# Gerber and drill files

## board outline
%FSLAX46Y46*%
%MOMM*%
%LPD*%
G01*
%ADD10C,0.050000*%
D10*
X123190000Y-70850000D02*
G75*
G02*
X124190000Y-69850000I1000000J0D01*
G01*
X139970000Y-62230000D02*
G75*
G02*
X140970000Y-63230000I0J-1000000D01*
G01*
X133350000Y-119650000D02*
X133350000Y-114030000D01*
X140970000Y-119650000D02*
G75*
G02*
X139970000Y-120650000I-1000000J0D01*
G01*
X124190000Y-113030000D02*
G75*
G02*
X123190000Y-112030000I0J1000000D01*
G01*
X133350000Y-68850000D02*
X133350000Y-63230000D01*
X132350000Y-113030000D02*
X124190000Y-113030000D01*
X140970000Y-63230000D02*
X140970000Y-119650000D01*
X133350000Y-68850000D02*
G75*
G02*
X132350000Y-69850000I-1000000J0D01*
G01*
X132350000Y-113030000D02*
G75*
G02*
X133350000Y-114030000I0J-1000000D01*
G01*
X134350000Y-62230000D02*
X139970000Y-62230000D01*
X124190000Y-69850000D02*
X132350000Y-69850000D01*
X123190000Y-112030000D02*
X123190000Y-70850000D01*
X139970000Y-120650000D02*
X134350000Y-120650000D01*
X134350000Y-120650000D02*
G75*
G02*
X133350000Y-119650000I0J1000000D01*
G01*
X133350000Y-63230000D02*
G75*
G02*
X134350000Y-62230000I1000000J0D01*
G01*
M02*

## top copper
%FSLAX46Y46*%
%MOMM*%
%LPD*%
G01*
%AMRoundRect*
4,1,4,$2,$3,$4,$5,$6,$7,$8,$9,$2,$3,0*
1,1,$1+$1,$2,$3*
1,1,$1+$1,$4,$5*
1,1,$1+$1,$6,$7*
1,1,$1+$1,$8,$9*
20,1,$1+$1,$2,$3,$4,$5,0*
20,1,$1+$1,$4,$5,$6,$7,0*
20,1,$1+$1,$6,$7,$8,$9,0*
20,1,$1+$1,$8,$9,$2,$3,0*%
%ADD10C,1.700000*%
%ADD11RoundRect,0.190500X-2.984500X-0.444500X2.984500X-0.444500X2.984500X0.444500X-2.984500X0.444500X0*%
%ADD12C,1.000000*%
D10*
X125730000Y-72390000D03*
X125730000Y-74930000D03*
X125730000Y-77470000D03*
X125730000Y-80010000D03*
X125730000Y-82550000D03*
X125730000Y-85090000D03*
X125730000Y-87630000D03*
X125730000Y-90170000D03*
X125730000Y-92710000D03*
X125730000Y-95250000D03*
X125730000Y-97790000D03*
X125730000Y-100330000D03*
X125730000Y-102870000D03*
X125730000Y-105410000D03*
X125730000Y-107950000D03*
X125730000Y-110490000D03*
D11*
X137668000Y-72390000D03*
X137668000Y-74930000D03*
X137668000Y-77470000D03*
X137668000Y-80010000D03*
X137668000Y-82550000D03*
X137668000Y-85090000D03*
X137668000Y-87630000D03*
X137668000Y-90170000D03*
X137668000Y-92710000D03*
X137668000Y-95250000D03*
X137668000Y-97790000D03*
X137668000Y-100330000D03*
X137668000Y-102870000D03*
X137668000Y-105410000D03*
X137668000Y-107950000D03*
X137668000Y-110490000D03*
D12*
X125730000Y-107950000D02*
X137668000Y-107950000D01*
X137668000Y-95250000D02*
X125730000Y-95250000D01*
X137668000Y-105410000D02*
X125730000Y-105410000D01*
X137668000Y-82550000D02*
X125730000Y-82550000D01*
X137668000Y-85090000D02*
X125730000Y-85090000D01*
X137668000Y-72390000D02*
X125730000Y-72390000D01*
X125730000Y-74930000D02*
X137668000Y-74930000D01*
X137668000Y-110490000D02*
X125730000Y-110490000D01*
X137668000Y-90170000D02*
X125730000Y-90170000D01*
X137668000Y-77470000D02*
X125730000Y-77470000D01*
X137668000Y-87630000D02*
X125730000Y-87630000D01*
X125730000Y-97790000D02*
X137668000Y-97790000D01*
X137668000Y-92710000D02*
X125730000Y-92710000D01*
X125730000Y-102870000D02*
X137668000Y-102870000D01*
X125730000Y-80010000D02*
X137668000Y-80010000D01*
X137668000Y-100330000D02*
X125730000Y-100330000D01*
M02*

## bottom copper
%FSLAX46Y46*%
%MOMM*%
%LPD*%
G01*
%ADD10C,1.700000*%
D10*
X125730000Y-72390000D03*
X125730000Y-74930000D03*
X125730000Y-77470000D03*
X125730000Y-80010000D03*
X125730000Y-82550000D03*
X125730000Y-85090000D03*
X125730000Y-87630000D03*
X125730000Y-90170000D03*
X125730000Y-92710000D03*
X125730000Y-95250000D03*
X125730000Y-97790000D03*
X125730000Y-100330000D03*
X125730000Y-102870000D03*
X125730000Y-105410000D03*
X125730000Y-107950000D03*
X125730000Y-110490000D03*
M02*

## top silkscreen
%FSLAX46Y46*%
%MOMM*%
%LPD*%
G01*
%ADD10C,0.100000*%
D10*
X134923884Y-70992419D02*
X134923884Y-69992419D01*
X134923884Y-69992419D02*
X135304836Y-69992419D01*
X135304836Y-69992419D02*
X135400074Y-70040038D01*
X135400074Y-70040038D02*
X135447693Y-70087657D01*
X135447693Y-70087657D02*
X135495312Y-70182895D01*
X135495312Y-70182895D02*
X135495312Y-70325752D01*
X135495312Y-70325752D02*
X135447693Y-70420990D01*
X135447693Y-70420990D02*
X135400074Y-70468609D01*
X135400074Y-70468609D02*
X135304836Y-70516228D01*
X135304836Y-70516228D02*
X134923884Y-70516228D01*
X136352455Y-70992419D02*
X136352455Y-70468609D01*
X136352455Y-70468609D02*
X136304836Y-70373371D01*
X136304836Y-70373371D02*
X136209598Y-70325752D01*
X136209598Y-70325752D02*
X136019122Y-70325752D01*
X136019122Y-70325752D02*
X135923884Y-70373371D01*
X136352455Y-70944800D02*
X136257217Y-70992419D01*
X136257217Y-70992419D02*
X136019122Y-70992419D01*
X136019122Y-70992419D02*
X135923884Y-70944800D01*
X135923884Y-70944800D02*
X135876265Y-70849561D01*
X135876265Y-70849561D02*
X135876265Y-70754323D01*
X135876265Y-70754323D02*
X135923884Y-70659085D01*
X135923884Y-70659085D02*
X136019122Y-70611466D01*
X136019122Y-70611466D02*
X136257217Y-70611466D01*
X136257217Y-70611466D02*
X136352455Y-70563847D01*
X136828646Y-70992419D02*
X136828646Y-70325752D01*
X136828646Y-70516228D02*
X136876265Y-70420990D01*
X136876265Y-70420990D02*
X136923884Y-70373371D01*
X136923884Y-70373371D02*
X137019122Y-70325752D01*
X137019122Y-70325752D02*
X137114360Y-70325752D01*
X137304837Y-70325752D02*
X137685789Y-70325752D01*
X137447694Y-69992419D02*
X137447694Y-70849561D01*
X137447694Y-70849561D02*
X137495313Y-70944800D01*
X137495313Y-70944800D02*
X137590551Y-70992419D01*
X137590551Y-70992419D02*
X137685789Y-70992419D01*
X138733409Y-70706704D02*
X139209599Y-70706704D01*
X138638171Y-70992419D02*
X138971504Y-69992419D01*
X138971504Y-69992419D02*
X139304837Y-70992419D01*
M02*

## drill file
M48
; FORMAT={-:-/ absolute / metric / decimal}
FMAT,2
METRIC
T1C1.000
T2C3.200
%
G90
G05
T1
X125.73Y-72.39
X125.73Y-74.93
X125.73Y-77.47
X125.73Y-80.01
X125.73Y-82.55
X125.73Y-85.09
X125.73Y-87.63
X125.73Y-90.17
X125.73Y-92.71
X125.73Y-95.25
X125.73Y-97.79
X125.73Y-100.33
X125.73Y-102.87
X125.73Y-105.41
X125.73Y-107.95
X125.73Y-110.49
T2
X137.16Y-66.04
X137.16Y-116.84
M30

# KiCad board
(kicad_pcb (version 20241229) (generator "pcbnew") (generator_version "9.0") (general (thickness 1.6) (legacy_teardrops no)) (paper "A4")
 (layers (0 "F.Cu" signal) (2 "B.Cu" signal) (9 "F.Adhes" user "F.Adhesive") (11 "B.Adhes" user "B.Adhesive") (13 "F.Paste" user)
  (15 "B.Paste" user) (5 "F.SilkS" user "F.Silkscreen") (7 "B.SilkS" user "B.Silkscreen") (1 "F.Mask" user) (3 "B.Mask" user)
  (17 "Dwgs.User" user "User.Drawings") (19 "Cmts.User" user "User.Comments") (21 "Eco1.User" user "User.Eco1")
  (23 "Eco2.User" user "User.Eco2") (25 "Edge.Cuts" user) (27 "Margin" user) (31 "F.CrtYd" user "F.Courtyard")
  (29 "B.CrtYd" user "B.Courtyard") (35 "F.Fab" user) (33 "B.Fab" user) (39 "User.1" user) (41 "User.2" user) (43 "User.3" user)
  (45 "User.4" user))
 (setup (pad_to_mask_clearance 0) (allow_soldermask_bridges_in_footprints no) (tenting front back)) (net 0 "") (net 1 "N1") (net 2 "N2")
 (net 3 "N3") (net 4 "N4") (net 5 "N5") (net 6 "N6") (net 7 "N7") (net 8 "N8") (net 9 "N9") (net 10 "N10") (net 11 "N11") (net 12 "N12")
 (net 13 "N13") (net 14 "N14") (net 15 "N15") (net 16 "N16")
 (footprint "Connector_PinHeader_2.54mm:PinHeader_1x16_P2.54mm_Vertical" (layer "F.Cu") (at 125.73 72.39)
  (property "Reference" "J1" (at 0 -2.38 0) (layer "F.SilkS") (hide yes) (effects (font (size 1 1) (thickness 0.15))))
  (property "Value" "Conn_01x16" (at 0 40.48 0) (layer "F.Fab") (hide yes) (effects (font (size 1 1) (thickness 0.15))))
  (pad "1" thru_hole circle (at 0 0) (size 1.7 1.7) (drill 1) (layers "*.Cu" "*.Mask") (remove_unused_layers no) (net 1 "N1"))
  (pad "2" thru_hole circle (at 0 2.54) (size 1.7 1.7) (drill 1) (layers "*.Cu" "*.Mask") (remove_unused_layers no) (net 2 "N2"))
  (pad "3" thru_hole circle (at 0 5.08) (size 1.7 1.7) (drill 1) (layers "*.Cu" "*.Mask") (remove_unused_layers no) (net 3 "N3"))
  (pad "4" thru_hole circle (at 0 7.62) (size 1.7 1.7) (drill 1) (layers "*.Cu" "*.Mask") (remove_unused_layers no) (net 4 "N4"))
  (pad "5" thru_hole circle (at 0 10.16) (size 1.7 1.7) (drill 1) (layers "*.Cu" "*.Mask") (remove_unused_layers no) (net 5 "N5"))
  (pad "6" thru_hole circle (at 0 12.7) (size 1.7 1.7) (drill 1) (layers "*.Cu" "*.Mask") (remove_unused_layers no) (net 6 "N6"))
  (pad "7" thru_hole circle (at 0 15.24) (size 1.7 1.7) (drill 1) (layers "*.Cu" "*.Mask") (remove_unused_layers no) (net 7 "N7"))
  (pad "8" thru_hole circle (at 0 17.78) (size 1.7 1.7) (drill 1) (layers "*.Cu" "*.Mask") (remove_unused_layers no) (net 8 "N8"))
  (pad "9" thru_hole circle (at 0 20.32) (size 1.7 1.7) (drill 1) (layers "*.Cu" "*.Mask") (remove_unused_layers no) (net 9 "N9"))
  (pad "10" thru_hole circle (at 0 22.86) (size 1.7 1.7) (drill 1) (layers "*.Cu" "*.Mask") (remove_unused_layers no) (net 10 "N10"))
  (pad "11" thru_hole circle (at 0 25.4) (size 1.7 1.7) (drill 1) (layers "*.Cu" "*.Mask") (remove_unused_layers no) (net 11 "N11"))
  (pad "12" thru_hole circle (at 0 27.94) (size 1.7 1.7) (drill 1) (layers "*.Cu" "*.Mask") (remove_unused_layers no) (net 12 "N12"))
  (pad "13" thru_hole circle (at 0 30.48) (size 1.7 1.7) (drill 1) (layers "*.Cu" "*.Mask") (remove_unused_layers no) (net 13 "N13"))
  (pad "14" thru_hole circle (at 0 33.02) (size 1.7 1.7) (drill 1) (layers "*.Cu" "*.Mask") (remove_unused_layers no) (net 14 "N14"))
  (pad "15" thru_hole circle (at 0 35.56) (size 1.7 1.7) (drill 1) (layers "*.Cu" "*.Mask") (remove_unused_layers no) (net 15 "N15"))
  (pad "16" thru_hole circle (at 0 38.1) (size 1.7 1.7) (drill 1) (layers "*.Cu" "*.Mask") (remove_unused_layers no) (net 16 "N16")))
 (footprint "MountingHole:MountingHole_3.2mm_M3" (layer "F.Cu") (at 137.16 116.84)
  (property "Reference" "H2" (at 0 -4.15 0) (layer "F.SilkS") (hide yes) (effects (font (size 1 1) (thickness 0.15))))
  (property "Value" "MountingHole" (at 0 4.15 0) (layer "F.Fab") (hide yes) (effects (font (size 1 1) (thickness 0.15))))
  (pad "" np_thru_hole circle (at 0 0) (size 3.2 3.2) (drill 3.2) (layers "*.Cu" "*.Mask")))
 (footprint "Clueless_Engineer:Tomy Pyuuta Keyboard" (layer "F.Cu") (at 137.668 72.39)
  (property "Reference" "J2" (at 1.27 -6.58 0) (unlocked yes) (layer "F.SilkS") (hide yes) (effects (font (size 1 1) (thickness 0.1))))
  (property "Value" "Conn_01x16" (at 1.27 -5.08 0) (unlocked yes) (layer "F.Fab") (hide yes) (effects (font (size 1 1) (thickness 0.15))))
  (pad "1" connect roundrect (at 0 0) (size 6.35 1.27) (layers "F.Cu" "F.Mask") (roundrect_rratio 0.15) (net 1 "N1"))
  (pad "2" connect roundrect (at 0 2.54) (size 6.35 1.27) (layers "F.Cu" "F.Mask") (roundrect_rratio 0.15) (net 2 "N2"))
  (pad "3" connect roundrect (at 0 5.08) (size 6.35 1.27) (layers "F.Cu" "F.Mask") (roundrect_rratio 0.15) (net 3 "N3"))
  (pad "4" connect roundrect (at 0 7.62) (size 6.35 1.27) (layers "F.Cu" "F.Mask") (roundrect_rratio 0.15) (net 4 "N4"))
  (pad "5" connect roundrect (at 0 10.16) (size 6.35 1.27) (layers "F.Cu" "F.Mask") (roundrect_rratio 0.15) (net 5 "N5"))
  (pad "6" connect roundrect (at 0 12.7) (size 6.35 1.27) (layers "F.Cu" "F.Mask") (roundrect_rratio 0.15) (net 6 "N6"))
  (pad "7" connect roundrect (at 0 15.24) (size 6.35 1.27) (layers "F.Cu" "F.Mask") (roundrect_rratio 0.15) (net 7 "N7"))
  (pad "8" connect roundrect (at 0 17.78) (size 6.35 1.27) (layers "F.Cu" "F.Mask") (roundrect_rratio 0.15) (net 8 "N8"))
  (pad "9" connect roundrect (at 0 20.32) (size 6.35 1.27) (layers "F.Cu" "F.Mask") (roundrect_rratio 0.15) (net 9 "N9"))
  (pad "10" connect roundrect (at 0 22.86) (size 6.35 1.27) (layers "F.Cu" "F.Mask") (roundrect_rratio 0.15) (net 10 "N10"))
  (pad "11" connect roundrect (at 0 25.4) (size 6.35 1.27) (layers "F.Cu" "F.Mask") (roundrect_rratio 0.15) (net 11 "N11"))
  (pad "12" connect roundrect (at 0 27.94) (size 6.35 1.27) (layers "F.Cu" "F.Mask") (roundrect_rratio 0.15) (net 12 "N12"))
  (pad "13" connect roundrect (at 0 30.48) (size 6.35 1.27) (layers "F.Cu" "F.Mask") (roundrect_rratio 0.15) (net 13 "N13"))
  (pad "14" connect roundrect (at 0 33.02) (size 6.35 1.27) (layers "F.Cu" "F.Mask") (roundrect_rratio 0.15) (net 14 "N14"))
  (pad "15" connect roundrect (at 0 35.56) (size 6.35 1.27) (layers "F.Cu" "F.Mask") (roundrect_rratio 0.15) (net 15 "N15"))
  (pad "16" connect roundrect (at 0 38.1) (size 6.35 1.27) (layers "F.Cu" "F.Mask") (roundrect_rratio 0.15) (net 16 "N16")))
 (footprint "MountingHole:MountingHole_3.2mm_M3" (layer "F.Cu") (at 137.16 66.04)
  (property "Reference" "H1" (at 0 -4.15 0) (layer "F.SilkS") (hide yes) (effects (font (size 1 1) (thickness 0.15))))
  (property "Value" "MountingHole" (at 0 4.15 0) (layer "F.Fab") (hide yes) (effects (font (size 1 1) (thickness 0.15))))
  (pad "" np_thru_hole circle (at 0 0) (size 3.2 3.2) (drill 3.2) (layers "*.Cu" "*.Mask")))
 (gr_arc (start 123.19 70.85) (mid 123.482893 70.142893) (end 124.19 69.85) (stroke (width 0.05) (type default)) (layer "Edge.Cuts"))
 (gr_arc (start 139.97 62.23) (mid 140.677107 62.522893) (end 140.97 63.23) (stroke (width 0.05) (type default)) (layer "Edge.Cuts"))
 (gr_line (start 133.35 119.65) (end 133.35 114.03) (stroke (width 0.05) (type default)) (layer "Edge.Cuts"))
 (gr_arc (start 140.97 119.65) (mid 140.677107 120.357107) (end 139.97 120.65) (stroke (width 0.05) (type default)) (layer "Edge.Cuts"))
 (gr_arc (start 124.19 113.03) (mid 123.482893 112.737107) (end 123.19 112.03) (stroke (width 0.05) (type default)) (layer "Edge.Cuts"))
 (gr_line (start 133.35 68.85) (end 133.35 63.23) (stroke (width 0.05) (type default)) (layer "Edge.Cuts"))
 (gr_line (start 132.35 113.03) (end 124.19 113.03) (stroke (width 0.05) (type default)) (layer "Edge.Cuts"))
 (gr_line (start 140.97 63.23) (end 140.97 119.65) (stroke (width 0.05) (type default)) (layer "Edge.Cuts"))
 (gr_arc (start 133.35 68.85) (mid 133.057107 69.557107) (end 132.35 69.85) (stroke (width 0.05) (type default)) (layer "Edge.Cuts"))
 (gr_arc (start 132.35 113.03) (mid 133.057107 113.322893) (end 133.35 114.03) (stroke (width 0.05) (type default)) (layer "Edge.Cuts"))
 (gr_line (start 134.35 62.23) (end 139.97 62.23) (stroke (width 0.05) (type default)) (layer "Edge.Cuts"))
 (gr_line (start 124.19 69.85) (end 132.35 69.85) (stroke (width 0.05) (type default)) (layer "Edge.Cuts"))
 (gr_line (start 123.19 112.03) (end 123.19 70.85) (stroke (width 0.05) (type default)) (layer "Edge.Cuts"))
 (gr_line (start 139.97 120.65) (end 134.35 120.65) (stroke (width 0.05) (type default)) (layer "Edge.Cuts"))
 (gr_arc (start 134.35 120.65) (mid 133.642893 120.357107) (end 133.35 119.65) (stroke (width 0.05) (type default)) (layer "Edge.Cuts"))
 (gr_arc (start 133.35 63.23) (mid 133.642893 62.522893) (end 134.35 62.23) (stroke (width 0.05) (type default)) (layer "Edge.Cuts"))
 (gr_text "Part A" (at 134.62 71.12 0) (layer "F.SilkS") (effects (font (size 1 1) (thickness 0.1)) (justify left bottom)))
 (segment (start 125.73 107.95) (end 137.668 107.95) (width 1) (layer "F.Cu") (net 15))
 (segment (start 137.668 95.25) (end 125.73 95.25) (width 1) (layer "F.Cu") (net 10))
 (segment (start 137.668 105.41) (end 125.73 105.41) (width 1) (layer "F.Cu") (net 14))
 (segment (start 137.668 82.55) (end 125.73 82.55) (width 1) (layer "F.Cu") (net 5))
 (segment (start 137.668 85.09) (end 125.73 85.09) (width 1) (layer "F.Cu") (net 6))
 (segment (start 137.668 72.39) (end 125.73 72.39) (width 1) (layer "F.Cu") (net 1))
 (segment (start 125.73 74.93) (end 137.668 74.93) (width 1) (layer "F.Cu") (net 2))
 (segment (start 137.668 110.49) (end 125.73 110.49) (width 1) (layer "F.Cu") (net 16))
 (segment (start 137.668 90.17) (end 125.73 90.17) (width 1) (layer "F.Cu") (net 8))
 (segment (start 137.668 77.47) (end 125.73 77.47) (width 1) (layer "F.Cu") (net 3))
 (segment (start 137.668 87.63) (end 125.73 87.63) (width 1) (layer "F.Cu") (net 7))
 (segment (start 125.73 97.79) (end 137.668 97.79) (width 1) (layer "F.Cu") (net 11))
 (segment (start 137.668 92.71) (end 125.73 92.71) (width 1) (layer "F.Cu") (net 9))
 (segment (start 125.73 102.87) (end 137.668 102.87) (width 1) (layer "F.Cu") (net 13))
 (segment (start 125.73 80.01) (end 137.668 80.01) (width 1) (layer "F.Cu") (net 4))
 (segment (start 137.668 100.33) (end 125.73 100.33) (width 1) (layer "F.Cu") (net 12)))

